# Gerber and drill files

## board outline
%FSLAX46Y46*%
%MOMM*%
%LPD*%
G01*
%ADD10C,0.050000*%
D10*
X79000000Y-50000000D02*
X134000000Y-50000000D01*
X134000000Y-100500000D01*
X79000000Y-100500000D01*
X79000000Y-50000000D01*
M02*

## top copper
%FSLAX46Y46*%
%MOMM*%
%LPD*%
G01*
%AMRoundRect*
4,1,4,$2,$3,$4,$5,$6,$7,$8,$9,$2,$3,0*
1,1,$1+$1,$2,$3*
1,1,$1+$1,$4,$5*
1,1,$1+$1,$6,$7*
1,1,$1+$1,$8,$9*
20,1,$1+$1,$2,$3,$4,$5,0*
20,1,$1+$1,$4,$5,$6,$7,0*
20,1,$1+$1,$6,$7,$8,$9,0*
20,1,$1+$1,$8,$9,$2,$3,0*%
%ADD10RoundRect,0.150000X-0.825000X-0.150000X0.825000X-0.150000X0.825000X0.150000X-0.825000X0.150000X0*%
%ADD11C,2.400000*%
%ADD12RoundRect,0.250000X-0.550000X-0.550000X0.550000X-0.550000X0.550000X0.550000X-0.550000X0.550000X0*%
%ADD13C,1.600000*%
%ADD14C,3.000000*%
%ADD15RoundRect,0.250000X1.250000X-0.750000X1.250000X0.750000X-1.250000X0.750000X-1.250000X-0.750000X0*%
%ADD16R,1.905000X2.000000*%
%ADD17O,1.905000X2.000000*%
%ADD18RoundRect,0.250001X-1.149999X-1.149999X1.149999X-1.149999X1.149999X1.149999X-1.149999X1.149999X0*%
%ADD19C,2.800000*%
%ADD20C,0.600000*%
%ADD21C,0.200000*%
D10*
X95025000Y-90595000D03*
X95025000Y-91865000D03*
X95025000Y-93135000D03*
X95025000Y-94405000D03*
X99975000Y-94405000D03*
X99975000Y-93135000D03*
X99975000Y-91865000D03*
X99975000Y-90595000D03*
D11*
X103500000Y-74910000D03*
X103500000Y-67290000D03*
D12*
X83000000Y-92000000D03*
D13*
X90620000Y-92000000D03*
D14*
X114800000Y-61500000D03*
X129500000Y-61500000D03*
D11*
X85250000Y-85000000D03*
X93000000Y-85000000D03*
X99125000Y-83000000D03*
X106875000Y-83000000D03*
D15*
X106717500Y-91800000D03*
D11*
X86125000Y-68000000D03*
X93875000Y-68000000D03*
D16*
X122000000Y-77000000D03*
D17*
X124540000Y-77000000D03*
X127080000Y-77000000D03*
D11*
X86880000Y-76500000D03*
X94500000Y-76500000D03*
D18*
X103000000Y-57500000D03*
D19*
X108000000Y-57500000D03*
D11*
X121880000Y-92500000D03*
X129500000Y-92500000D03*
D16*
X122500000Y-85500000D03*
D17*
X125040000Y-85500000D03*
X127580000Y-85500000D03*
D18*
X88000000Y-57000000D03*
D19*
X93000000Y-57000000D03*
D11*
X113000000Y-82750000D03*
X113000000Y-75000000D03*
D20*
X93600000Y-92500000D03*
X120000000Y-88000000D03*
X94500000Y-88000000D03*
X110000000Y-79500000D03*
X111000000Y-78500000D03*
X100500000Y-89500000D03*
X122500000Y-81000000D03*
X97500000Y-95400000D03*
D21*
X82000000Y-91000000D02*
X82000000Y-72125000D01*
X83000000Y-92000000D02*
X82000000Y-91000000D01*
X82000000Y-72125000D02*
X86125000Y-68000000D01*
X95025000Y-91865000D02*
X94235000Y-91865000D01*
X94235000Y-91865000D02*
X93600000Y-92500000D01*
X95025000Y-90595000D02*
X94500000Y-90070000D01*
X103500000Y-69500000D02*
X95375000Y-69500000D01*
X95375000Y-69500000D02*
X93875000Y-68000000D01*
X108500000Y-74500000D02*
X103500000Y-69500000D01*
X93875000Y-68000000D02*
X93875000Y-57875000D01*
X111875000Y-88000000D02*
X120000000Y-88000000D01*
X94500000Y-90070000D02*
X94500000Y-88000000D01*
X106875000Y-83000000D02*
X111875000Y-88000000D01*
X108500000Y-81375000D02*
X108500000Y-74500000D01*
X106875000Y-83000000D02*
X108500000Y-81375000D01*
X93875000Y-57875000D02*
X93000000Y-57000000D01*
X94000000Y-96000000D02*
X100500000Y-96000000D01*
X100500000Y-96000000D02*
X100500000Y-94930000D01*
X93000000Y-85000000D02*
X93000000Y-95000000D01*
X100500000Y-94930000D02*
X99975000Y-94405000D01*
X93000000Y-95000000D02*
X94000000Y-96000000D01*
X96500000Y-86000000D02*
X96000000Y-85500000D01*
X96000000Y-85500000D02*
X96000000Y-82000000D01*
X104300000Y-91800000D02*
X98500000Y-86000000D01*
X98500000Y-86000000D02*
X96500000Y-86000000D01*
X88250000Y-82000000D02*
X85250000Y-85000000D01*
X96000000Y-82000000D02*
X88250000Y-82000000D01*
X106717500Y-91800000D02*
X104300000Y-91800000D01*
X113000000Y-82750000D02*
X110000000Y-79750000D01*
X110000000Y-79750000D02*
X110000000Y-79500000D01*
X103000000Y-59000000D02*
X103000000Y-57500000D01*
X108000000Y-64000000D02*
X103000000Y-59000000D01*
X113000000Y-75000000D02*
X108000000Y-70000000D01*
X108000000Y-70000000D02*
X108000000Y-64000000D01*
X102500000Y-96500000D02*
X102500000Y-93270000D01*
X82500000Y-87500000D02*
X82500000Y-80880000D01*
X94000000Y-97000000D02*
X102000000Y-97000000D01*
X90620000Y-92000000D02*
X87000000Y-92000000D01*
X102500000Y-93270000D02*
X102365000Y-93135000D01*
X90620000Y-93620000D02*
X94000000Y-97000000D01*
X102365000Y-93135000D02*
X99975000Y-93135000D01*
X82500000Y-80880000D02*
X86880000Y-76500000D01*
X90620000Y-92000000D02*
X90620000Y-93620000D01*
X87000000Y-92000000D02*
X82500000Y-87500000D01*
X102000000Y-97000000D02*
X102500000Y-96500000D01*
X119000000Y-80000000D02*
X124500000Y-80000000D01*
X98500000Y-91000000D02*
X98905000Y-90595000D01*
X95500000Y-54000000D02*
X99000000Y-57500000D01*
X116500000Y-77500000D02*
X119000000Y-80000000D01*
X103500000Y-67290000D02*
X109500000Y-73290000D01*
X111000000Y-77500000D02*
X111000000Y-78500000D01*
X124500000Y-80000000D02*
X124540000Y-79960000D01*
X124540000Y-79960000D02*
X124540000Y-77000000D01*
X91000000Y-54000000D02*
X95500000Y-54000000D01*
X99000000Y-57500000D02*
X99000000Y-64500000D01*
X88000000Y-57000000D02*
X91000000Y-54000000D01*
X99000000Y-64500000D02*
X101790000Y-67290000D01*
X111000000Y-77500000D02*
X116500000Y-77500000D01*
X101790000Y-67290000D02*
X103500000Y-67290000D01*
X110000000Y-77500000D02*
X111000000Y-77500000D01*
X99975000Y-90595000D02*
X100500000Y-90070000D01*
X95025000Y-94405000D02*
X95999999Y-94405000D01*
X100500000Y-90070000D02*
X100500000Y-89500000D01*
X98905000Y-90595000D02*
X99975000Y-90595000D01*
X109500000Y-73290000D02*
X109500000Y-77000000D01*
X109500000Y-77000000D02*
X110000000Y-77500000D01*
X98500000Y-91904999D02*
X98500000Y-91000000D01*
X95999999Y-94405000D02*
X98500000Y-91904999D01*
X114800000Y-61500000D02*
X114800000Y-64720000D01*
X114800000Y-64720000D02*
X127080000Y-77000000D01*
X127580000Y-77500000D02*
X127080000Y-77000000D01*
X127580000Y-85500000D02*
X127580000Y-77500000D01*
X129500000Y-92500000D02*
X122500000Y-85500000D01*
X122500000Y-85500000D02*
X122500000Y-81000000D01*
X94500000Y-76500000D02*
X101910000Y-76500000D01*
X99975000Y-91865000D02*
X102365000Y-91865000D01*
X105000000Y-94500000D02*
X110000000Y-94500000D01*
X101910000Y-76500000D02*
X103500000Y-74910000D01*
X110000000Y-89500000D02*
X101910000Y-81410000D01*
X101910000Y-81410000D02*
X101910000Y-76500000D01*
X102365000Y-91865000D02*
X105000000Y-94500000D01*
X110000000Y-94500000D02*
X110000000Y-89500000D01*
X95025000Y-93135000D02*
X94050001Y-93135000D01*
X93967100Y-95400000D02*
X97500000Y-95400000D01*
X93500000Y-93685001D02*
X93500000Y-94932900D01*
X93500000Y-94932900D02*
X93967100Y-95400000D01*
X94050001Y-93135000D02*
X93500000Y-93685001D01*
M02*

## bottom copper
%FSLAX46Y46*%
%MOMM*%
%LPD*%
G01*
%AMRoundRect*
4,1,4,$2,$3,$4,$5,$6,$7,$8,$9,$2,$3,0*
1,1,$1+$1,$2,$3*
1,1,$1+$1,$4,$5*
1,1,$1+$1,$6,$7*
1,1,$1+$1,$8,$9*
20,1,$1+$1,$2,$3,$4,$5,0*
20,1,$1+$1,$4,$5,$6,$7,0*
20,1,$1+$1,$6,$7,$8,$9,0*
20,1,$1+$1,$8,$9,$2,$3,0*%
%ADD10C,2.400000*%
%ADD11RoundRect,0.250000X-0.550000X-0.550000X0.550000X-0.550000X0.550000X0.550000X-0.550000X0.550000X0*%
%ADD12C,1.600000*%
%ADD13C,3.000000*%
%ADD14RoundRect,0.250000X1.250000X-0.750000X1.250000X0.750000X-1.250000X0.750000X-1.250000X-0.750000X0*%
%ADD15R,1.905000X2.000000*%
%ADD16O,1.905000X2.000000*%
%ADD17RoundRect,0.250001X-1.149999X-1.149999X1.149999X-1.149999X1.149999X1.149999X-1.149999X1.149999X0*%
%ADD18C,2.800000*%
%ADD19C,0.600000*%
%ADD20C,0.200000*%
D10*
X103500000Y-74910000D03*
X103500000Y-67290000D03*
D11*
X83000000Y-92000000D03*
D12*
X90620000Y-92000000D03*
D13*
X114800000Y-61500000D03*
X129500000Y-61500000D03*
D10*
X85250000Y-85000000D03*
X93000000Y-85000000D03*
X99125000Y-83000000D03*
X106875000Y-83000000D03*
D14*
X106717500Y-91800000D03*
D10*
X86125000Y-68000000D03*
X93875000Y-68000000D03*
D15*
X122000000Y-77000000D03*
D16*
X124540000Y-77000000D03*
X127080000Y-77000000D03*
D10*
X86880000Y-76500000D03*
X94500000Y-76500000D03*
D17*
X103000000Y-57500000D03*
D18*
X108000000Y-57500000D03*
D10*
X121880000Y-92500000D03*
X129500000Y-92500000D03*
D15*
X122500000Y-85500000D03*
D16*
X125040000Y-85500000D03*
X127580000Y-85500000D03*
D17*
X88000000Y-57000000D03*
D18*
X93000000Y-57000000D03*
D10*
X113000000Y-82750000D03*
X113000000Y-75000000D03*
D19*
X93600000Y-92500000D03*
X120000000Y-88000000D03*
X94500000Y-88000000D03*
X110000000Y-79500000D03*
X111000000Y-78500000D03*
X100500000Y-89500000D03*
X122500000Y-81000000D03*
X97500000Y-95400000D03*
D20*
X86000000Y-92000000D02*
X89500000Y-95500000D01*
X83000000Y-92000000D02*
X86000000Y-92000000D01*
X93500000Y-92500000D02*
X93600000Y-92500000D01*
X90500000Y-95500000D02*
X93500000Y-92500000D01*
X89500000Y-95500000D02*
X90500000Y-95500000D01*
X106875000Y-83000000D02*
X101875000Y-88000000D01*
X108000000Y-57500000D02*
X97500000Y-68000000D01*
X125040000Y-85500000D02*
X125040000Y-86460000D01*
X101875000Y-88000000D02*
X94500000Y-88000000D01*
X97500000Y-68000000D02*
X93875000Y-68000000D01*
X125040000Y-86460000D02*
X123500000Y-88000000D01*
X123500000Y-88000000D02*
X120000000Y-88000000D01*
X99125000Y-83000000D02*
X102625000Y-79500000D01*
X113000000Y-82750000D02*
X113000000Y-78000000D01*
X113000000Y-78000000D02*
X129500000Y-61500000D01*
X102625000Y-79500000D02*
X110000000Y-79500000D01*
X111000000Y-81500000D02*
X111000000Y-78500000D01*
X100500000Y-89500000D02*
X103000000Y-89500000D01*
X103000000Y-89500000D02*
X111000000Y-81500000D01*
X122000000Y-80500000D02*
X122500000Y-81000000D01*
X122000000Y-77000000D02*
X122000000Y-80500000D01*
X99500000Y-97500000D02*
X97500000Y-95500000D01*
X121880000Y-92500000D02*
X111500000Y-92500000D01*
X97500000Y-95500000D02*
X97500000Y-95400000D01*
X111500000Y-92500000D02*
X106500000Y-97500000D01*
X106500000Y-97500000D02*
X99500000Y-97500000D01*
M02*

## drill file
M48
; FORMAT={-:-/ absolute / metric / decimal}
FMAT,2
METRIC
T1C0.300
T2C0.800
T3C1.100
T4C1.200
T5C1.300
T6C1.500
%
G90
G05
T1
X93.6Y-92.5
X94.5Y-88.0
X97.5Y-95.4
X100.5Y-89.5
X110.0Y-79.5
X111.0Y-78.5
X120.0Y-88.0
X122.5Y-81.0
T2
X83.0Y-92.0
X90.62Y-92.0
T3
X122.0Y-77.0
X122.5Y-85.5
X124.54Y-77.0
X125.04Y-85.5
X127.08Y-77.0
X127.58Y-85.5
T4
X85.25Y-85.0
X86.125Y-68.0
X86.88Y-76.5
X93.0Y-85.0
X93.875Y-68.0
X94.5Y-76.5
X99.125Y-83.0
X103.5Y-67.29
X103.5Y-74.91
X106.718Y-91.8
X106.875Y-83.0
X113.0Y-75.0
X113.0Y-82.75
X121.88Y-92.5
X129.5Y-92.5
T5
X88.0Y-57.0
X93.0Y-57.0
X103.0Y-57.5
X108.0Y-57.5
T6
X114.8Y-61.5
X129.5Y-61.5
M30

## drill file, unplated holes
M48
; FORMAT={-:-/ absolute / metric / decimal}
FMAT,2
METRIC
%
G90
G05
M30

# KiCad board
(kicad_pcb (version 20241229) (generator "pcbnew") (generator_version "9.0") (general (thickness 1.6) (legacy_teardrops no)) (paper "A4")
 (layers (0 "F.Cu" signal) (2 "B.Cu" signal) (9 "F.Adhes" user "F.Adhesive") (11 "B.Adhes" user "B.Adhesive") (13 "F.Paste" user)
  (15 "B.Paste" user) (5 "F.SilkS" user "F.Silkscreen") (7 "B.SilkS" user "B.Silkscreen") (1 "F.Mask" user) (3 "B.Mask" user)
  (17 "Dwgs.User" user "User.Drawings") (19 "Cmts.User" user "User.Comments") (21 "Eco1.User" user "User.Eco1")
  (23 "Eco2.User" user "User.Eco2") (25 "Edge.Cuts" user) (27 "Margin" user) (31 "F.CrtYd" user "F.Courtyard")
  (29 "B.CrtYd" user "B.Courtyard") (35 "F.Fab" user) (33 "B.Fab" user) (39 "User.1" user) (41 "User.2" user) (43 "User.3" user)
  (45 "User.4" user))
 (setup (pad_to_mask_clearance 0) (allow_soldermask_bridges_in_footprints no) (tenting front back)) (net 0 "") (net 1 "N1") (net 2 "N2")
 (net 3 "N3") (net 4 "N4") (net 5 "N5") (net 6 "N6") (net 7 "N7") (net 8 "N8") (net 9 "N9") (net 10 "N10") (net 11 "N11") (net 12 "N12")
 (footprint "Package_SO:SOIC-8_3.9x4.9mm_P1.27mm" (layer "F.Cu") (at 97.5 92.5)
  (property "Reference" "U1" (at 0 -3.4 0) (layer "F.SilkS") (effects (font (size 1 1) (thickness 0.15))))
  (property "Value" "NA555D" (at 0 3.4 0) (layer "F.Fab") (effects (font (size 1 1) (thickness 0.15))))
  (pad "1" smd roundrect (at -2.475 -1.905) (size 1.95 0.6) (layers "F.Cu" "F.Mask" "F.Paste") (roundrect_rratio 0.25) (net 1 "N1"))
  (pad "2" smd roundrect (at -2.475 -0.635) (size 1.95 0.6) (layers "F.Cu" "F.Mask" "F.Paste") (roundrect_rratio 0.25) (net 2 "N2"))
  (pad "3" smd roundrect (at -2.475 0.635) (size 1.95 0.6) (layers "F.Cu" "F.Mask" "F.Paste") (roundrect_rratio 0.25) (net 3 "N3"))
  (pad "4" smd roundrect (at -2.475 1.905) (size 1.95 0.6) (layers "F.Cu" "F.Mask" "F.Paste") (roundrect_rratio 0.25) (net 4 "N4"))
  (pad "5" smd roundrect (at 2.475 1.905) (size 1.95 0.6) (layers "F.Cu" "F.Mask" "F.Paste") (roundrect_rratio 0.25) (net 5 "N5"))
  (pad "6" smd roundrect (at 2.475 0.635) (size 1.95 0.6) (layers "F.Cu" "F.Mask" "F.Paste") (roundrect_rratio 0.25) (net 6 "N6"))
  (pad "7" smd roundrect (at 2.475 -0.635) (size 1.95 0.6) (layers "F.Cu" "F.Mask" "F.Paste") (roundrect_rratio 0.25) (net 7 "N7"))
  (pad "8" smd roundrect (at 2.475 -1.905) (size 1.95 0.6) (layers "F.Cu" "F.Mask" "F.Paste") (roundrect_rratio 0.25) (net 4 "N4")))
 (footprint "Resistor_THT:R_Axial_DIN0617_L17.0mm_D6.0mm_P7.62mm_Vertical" (layer "F.Cu") (at 103.5 74.91 90)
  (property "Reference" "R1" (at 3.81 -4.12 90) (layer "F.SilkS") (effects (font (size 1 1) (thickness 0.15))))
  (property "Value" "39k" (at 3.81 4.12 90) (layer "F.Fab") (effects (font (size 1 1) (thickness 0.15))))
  (pad "1" thru_hole circle (at 0 0 90) (size 2.4 2.4) (drill 1.2) (layers "*.Cu" "*.Mask") (remove_unused_layers no) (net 7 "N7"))
  (pad "2" thru_hole circle (at 7.62 0 90) (size 2.4 2.4) (drill 1.2) (layers "*.Cu" "*.Mask") (remove_unused_layers no) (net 4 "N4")))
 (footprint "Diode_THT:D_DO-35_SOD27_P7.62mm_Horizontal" (layer "F.Cu") (at 83 92)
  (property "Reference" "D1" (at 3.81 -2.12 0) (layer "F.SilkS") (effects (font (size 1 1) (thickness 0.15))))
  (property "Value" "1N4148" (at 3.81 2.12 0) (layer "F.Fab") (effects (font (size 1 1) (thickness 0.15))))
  (pad "1" thru_hole roundrect (at 0 0) (size 1.6 1.6) (drill 0.8) (layers "*.Cu" "*.Mask") (remove_unused_layers no)
   (roundrect_rratio 0.15625) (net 2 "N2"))
  (pad "2" thru_hole circle (at 7.62 0) (size 1.6 1.6) (drill 0.8) (layers "*.Cu" "*.Mask") (remove_unused_layers no) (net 6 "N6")))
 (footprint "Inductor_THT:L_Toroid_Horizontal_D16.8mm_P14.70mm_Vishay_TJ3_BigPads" (layer "F.Cu") (at 114.8 61.5)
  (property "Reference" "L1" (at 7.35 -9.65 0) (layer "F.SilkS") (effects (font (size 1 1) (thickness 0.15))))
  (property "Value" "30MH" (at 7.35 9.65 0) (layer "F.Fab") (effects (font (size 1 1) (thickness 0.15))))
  (pad "1" thru_hole circle (at 0 0) (size 3 3) (drill 1.5) (layers "*.Cu" "*.Mask") (remove_unused_layers no) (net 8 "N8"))
  (pad "2" thru_hole circle (at 14.7 0) (size 3 3) (drill 1.5) (layers "*.Cu" "*.Mask") (remove_unused_layers no) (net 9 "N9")))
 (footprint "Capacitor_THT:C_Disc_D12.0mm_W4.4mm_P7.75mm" (layer "F.Cu") (at 85.25 85)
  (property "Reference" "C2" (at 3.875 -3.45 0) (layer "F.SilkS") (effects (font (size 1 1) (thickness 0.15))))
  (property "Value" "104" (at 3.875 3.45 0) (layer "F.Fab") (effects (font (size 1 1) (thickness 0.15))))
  (pad "1" thru_hole circle (at 0 0) (size 2.4 2.4) (drill 1.2) (layers "*.Cu" "*.Mask") (remove_unused_layers no) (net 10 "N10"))
  (pad "2" thru_hole circle (at 7.75 0) (size 2.4 2.4) (drill 1.2) (layers "*.Cu" "*.Mask") (remove_unused_layers no) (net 5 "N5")))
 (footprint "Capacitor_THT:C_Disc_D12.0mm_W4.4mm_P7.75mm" (layer "F.Cu") (at 99.125 83)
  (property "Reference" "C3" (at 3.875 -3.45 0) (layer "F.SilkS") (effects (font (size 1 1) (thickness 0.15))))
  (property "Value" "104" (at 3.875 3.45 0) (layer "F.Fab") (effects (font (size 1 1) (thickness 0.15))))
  (pad "1" thru_hole circle (at 0 0) (size 2.4 2.4) (drill 1.2) (layers "*.Cu" "*.Mask") (remove_unused_layers no) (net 9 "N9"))
  (pad "2" thru_hole circle (at 7.75 0) (size 2.4 2.4) (drill 1.2) (layers "*.Cu" "*.Mask") (remove_unused_layers no) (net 1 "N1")))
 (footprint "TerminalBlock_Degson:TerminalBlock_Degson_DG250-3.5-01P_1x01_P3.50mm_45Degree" (layer "F.Cu") (at 106.7175 91.8 90)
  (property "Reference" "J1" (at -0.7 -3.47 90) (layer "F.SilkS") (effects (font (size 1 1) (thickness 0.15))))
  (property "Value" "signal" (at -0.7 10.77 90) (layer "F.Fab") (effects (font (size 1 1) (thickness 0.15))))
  (pad "1" thru_hole roundrect (at 0 0 90) (size 2 3) (drill 1.2) (layers "*.Cu" "*.Mask") (remove_unused_layers no)
   (roundrect_rratio 0.125) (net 10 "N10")))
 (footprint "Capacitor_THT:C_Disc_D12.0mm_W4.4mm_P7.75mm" (layer "F.Cu") (at 86.125 68)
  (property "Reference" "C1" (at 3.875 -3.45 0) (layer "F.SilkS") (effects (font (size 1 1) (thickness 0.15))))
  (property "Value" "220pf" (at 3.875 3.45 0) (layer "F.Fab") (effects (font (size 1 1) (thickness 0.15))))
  (pad "1" thru_hole circle (at 0 0) (size 2.4 2.4) (drill 1.2) (layers "*.Cu" "*.Mask") (remove_unused_layers no) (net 2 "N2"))
  (pad "2" thru_hole circle (at 7.75 0) (size 2.4 2.4) (drill 1.2) (layers "*.Cu" "*.Mask") (remove_unused_layers no) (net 1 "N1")))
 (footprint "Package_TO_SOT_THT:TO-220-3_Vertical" (layer "F.Cu") (at 122 77)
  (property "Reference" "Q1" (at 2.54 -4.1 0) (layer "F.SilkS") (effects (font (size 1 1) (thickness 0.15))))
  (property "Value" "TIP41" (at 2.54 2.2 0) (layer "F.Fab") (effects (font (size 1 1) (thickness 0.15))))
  (pad "1" thru_hole rect (at 0 0) (size 1.905 2) (drill 1.1) (layers "*.Cu" "*.Mask") (remove_unused_layers no) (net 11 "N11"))
  (pad "2" thru_hole oval (at 2.54 0) (size 1.905 2) (drill 1.1) (layers "*.Cu" "*.Mask") (remove_unused_layers no) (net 4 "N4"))
  (pad "3" thru_hole oval (at 5.08 0) (size 1.905 2) (drill 1.1) (layers "*.Cu" "*.Mask") (remove_unused_layers no) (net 8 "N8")))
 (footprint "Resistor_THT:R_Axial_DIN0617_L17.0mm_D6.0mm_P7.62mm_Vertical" (layer "F.Cu") (at 86.88 76.5)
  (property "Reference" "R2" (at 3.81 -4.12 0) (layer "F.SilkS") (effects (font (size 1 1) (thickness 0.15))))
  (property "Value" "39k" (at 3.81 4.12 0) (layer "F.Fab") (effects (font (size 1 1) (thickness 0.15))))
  (pad "1" thru_hole circle (at 0 0) (size 2.4 2.4) (drill 1.2) (layers "*.Cu" "*.Mask") (remove_unused_layers no) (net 6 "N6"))
  (pad "2" thru_hole circle (at 7.62 0) (size 2.4 2.4) (drill 1.2) (layers "*.Cu" "*.Mask") (remove_unused_layers no) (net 7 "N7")))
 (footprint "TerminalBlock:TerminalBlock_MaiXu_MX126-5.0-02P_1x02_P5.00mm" (layer "F.Cu") (at 103 57.5)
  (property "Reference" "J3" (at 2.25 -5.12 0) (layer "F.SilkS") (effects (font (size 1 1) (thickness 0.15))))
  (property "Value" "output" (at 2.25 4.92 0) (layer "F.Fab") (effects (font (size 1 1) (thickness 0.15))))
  (pad "1" thru_hole roundrect (at 0 0) (size 2.8 2.8) (drill 1.3) (layers "*.Cu" "*.Mask") (remove_unused_layers no)
   (roundrect_rratio 0.089286) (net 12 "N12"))
  (pad "2" thru_hole circle (at 5 0) (size 2.8 2.8) (drill 1.3) (layers "*.Cu" "*.Mask") (remove_unused_layers no) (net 1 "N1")))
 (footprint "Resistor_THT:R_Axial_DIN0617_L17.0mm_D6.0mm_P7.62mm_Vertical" (layer "F.Cu") (at 121.88 92.5)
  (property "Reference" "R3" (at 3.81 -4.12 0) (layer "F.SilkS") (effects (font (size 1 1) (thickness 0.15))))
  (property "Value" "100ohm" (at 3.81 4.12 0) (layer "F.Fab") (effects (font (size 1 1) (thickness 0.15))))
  (pad "1" thru_hole circle (at 0 0) (size 2.4 2.4) (drill 1.2) (layers "*.Cu" "*.Mask") (remove_unused_layers no) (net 3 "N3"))
  (pad "2" thru_hole circle (at 7.62 0) (size 2.4 2.4) (drill 1.2) (layers "*.Cu" "*.Mask") (remove_unused_layers no) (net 11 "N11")))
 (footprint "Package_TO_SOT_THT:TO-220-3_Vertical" (layer "F.Cu") (at 122.5 85.5)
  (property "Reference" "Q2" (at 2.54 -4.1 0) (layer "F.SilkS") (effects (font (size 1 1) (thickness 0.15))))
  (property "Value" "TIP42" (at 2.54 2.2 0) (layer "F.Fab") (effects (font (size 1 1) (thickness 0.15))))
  (pad "1" thru_hole rect (at 0 0) (size 1.905 2) (drill 1.1) (layers "*.Cu" "*.Mask") (remove_unused_layers no) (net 11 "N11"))
  (pad "2" thru_hole oval (at 2.54 0) (size 1.905 2) (drill 1.1) (layers "*.Cu" "*.Mask") (remove_unused_layers no) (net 1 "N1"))
  (pad "3" thru_hole oval (at 5.08 0) (size 1.905 2) (drill 1.1) (layers "*.Cu" "*.Mask") (remove_unused_layers no) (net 8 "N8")))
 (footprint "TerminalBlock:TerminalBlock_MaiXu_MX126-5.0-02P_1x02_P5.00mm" (layer "F.Cu") (at 88 57)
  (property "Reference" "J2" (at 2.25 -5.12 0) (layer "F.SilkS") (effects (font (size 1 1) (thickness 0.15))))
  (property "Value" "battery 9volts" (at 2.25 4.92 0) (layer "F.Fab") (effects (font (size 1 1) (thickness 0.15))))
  (pad "1" thru_hole roundrect (at 0 0) (size 2.8 2.8) (drill 1.3) (layers "*.Cu" "*.Mask") (remove_unused_layers no)
   (roundrect_rratio 0.089286) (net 4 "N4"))
  (pad "2" thru_hole circle (at 5 0) (size 2.8 2.8) (drill 1.3) (layers "*.Cu" "*.Mask") (remove_unused_layers no) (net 1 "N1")))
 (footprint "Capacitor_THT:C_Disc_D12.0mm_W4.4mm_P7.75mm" (layer "F.Cu") (at 113 82.75 90)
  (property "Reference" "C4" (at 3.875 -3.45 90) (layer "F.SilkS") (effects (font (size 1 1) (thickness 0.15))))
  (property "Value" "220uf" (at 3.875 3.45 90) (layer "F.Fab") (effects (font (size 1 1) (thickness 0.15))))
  (pad "1" thru_hole circle (at 0 0 90) (size 2.4 2.4) (drill 1.2) (layers "*.Cu" "*.Mask") (remove_unused_layers no) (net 9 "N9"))
  (pad "2" thru_hole circle (at 7.75 0 90) (size 2.4 2.4) (drill 1.2) (layers "*.Cu" "*.Mask") (remove_unused_layers no) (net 12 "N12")))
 (gr_rect (start 79 50) (end 134 100.5) (stroke (width 0.05) (type default)) (fill no) (layer "Edge.Cuts"))
 (segment (start 82 91) (end 82 72.125) (width 0.2) (layer "F.Cu") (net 2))
 (segment (start 83 92) (end 82 91) (width 0.2) (layer "F.Cu") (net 2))
 (segment (start 82 72.125) (end 86.125 68) (width 0.2) (layer "F.Cu") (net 2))
 (segment (start 95.025 91.865) (end 94.235 91.865) (width 0.2) (layer "F.Cu") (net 2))
 (segment (start 94.235 91.865) (end 93.6 92.5) (width 0.2) (layer "F.Cu") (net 2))
 (via (at 93.6 92.5) (size 0.6) (drill 0.3) (layers "F.Cu" "B.Cu") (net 2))
 (segment (start 86 92) (end 89.5 95.5) (width 0.2) (layer "B.Cu") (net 2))
 (segment (start 83 92) (end 86 92) (width 0.2) (layer "B.Cu") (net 2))
 (segment (start 93.5 92.5) (end 93.6 92.5) (width 0.2) (layer "B.Cu") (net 2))
 (segment (start 90.5 95.5) (end 93.5 92.5) (width 0.2) (layer "B.Cu") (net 2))
 (segment (start 89.5 95.5) (end 90.5 95.5) (width 0.2) (layer "B.Cu") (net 2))
 (segment (start 95.025 90.595) (end 94.5 90.07) (width 0.2) (layer "F.Cu") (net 1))
 (segment (start 103.5 69.5) (end 95.375 69.5) (width 0.2) (layer "F.Cu") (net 1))
 (segment (start 95.375 69.5) (end 93.875 68) (width 0.2) (layer "F.Cu") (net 1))
 (segment (start 108.5 74.5) (end 103.5 69.5) (width 0.2) (layer "F.Cu") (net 1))
 (segment (start 93.875 68) (end 93.875 57.875) (width 0.2) (layer "F.Cu") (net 1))
 (segment (start 111.875 88) (end 120 88) (width 0.2) (layer "F.Cu") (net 1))
 (segment (start 94.5 90.07) (end 94.5 88) (width 0.2) (layer "F.Cu") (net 1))
 (segment (start 106.875 83) (end 111.875 88) (width 0.2) (layer "F.Cu") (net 1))
 (segment (start 108.5 81.375) (end 108.5 74.5) (width 0.2) (layer "F.Cu") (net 1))
 (segment (start 106.875 83) (end 108.5 81.375) (width 0.2) (layer "F.Cu") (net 1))
 (segment (start 93.875 57.875) (end 93 57) (width 0.2) (layer "F.Cu") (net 1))
 (via (at 120 88) (size 0.6) (drill 0.3) (layers "F.Cu" "B.Cu") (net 1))
 (via (at 94.5 88) (size 0.6) (drill 0.3) (layers "F.Cu" "B.Cu") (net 1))
 (segment (start 106.875 83) (end 101.875 88) (width 0.2) (layer "B.Cu") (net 1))
 (segment (start 108 57.5) (end 97.5 68) (width 0.2) (layer "B.Cu") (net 1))
 (segment (start 125.04 85.5) (end 125.04 86.46) (width 0.2) (layer "B.Cu") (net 1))
 (segment (start 101.875 88) (end 94.5 88) (width 0.2) (layer "B.Cu") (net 1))
 (segment (start 97.5 68) (end 93.875 68) (width 0.2) (layer "B.Cu") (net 1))
 (segment (start 125.04 86.46) (end 123.5 88) (width 0.2) (layer "B.Cu") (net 1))
 (segment (start 123.5 88) (end 120 88) (width 0.2) (layer "B.Cu") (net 1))
 (segment (start 94 96) (end 100.5 96) (width 0.2) (layer "F.Cu") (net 5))
 (segment (start 100.5 96) (end 100.5 94.93) (width 0.2) (layer "F.Cu") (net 5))
 (segment (start 93 85) (end 93 95) (width 0.2) (layer "F.Cu") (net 5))
 (segment (start 100.5 94.93) (end 99.975 94.405) (width 0.2) (layer "F.Cu") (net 5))
 (segment (start 93 95) (end 94 96) (width 0.2) (layer "F.Cu") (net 5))
 (segment (start 96.5 86) (end 96 85.5) (width 0.2) (layer "F.Cu") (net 10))
 (segment (start 96 85.5) (end 96 82) (width 0.2) (layer "F.Cu") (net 10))
 (segment (start 104.3 91.8) (end 98.5 86) (width 0.2) (layer "F.Cu") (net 10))
 (segment (start 98.5 86) (end 96.5 86) (width 0.2) (layer "F.Cu") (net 10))
 (segment (start 88.25 82) (end 85.25 85) (width 0.2) (layer "F.Cu") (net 10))
 (segment (start 96 82) (end 88.25 82) (width 0.2) (layer "F.Cu") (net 10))
 (segment (start 106.7175 91.8) (end 104.3 91.8) (width 0.2) (layer "F.Cu") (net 10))
 (segment (start 113 82.75) (end 110 79.75) (width 0.2) (layer "F.Cu") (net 9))
 (segment (start 110 79.75) (end 110 79.5) (width 0.2) (layer "F.Cu") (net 9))
 (via (at 110 79.5) (size 0.6) (drill 0.3) (layers "F.Cu" "B.Cu") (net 9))
 (segment (start 99.125 83) (end 102.625 79.5) (width 0.2) (layer "B.Cu") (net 9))
 (segment (start 113 82.75) (end 113 78) (width 0.2) (layer "B.Cu") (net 9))
 (segment (start 113 78) (end 129.5 61.5) (width 0.2) (layer "B.Cu") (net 9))
 (segment (start 102.625 79.5) (end 110 79.5) (width 0.2) (layer "B.Cu") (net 9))
 (segment (start 103 59) (end 103 57.5) (width 0.2) (layer "F.Cu") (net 12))
 (segment (start 108 64) (end 103 59) (width 0.2) (layer "F.Cu") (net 12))
 (segment (start 113 75) (end 108 70) (width 0.2) (layer "F.Cu") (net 12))
 (segment (start 108 70) (end 108 64) (width 0.2) (layer "F.Cu") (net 12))
 (segment (start 102.5 96.5) (end 102.5 93.27) (width 0.2) (layer "F.Cu") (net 6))
 (segment (start 82.5 87.5) (end 82.5 80.88) (width 0.2) (layer "F.Cu") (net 6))
 (segment (start 94 97) (end 102 97) (width 0.2) (layer "F.Cu") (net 6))
 (segment (start 90.62 92) (end 87 92) (width 0.2) (layer "F.Cu") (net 6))
 (segment (start 102.5 93.27) (end 102.365 93.135) (width 0.2) (layer "F.Cu") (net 6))
 (segment (start 90.62 93.62) (end 94 97) (width 0.2) (layer "F.Cu") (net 6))
 (segment (start 102.365 93.135) (end 99.975 93.135) (width 0.2) (layer "F.Cu") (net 6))
 (segment (start 82.5 80.88) (end 86.88 76.5) (width 0.2) (layer "F.Cu") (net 6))
 (segment (start 90.62 92) (end 90.62 93.62) (width 0.2) (layer "F.Cu") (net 6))
 (segment (start 87 92) (end 82.5 87.5) (width 0.2) (layer "F.Cu") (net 6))
 (segment (start 102 97) (end 102.5 96.5) (width 0.2) (layer "F.Cu") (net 6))
 (segment (start 119 80) (end 124.5 80) (width 0.2) (layer "F.Cu") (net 4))
 (segment (start 98.5 91) (end 98.905 90.595) (width 0.2) (layer "F.Cu") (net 4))
 (segment (start 95.5 54) (end 99 57.5) (width 0.2) (layer "F.Cu") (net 4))
 (segment (start 116.5 77.5) (end 119 80) (width 0.2) (layer "F.Cu") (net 4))
 (segment (start 103.5 67.29) (end 109.5 73.29) (width 0.2) (layer "F.Cu") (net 4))
 (segment (start 111 77.5) (end 111 78.5) (width 0.2) (layer "F.Cu") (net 4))
 (segment (start 124.5 80) (end 124.54 79.96) (width 0.2) (layer "F.Cu") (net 4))
 (segment (start 124.54 79.96) (end 124.54 77) (width 0.2) (layer "F.Cu") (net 4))
 (segment (start 91 54) (end 95.5 54) (width 0.2) (layer "F.Cu") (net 4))
 (segment (start 99 57.5) (end 99 64.5) (width 0.2) (layer "F.Cu") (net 4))
 (segment (start 88 57) (end 91 54) (width 0.2) (layer "F.Cu") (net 4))
 (segment (start 99 64.5) (end 101.79 67.29) (width 0.2) (layer "F.Cu") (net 4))
 (segment (start 111 77.5) (end 116.5 77.5) (width 0.2) (layer "F.Cu") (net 4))
 (segment (start 101.79 67.29) (end 103.5 67.29) (width 0.2) (layer "F.Cu") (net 4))
 (segment (start 110 77.5) (end 111 77.5) (width 0.2) (layer "F.Cu") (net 4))
 (segment (start 99.975 90.595) (end 100.5 90.07) (width 0.2) (layer "F.Cu") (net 4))
 (segment (start 95.025 94.405) (end 95.999999 94.405) (width 0.2) (layer "F.Cu") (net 4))
 (segment (start 100.5 90.07) (end 100.5 89.5) (width 0.2) (layer "F.Cu") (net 4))
 (segment (start 98.905 90.595) (end 99.975 90.595) (width 0.2) (layer "F.Cu") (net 4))
 (segment (start 109.5 73.29) (end 109.5 77) (width 0.2) (layer "F.Cu") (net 4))
 (segment (start 109.5 77) (end 110 77.5) (width 0.2) (layer "F.Cu") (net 4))
 (segment (start 98.5 91.904999) (end 98.5 91) (width 0.2) (layer "F.Cu") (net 4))
 (segment (start 95.999999 94.405) (end 98.5 91.904999) (width 0.2) (layer "F.Cu") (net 4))
 (via (at 111 78.5) (size 0.6) (drill 0.3) (layers "F.Cu" "B.Cu") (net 4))
 (via (at 100.5 89.5) (size 0.6) (drill 0.3) (layers "F.Cu" "B.Cu") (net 4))
 (segment (start 111 81.5) (end 111 78.5) (width 0.2) (layer "B.Cu") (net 4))
 (segment (start 100.5 89.5) (end 103 89.5) (width 0.2) (layer "B.Cu") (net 4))
 (segment (start 103 89.5) (end 111 81.5) (width 0.2) (layer "B.Cu") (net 4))
 (segment (start 114.8 61.5) (end 114.8 64.72) (width 0.2) (layer "F.Cu") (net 8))
 (segment (start 114.8 64.72) (end 127.08 77) (width 0.2) (layer "F.Cu") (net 8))
 (segment (start 127.58 77.5) (end 127.08 77) (width 0.2) (layer "F.Cu") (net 8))
 (segment (start 127.58 85.5) (end 127.58 77.5) (width 0.2) (layer "F.Cu") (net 8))
 (segment (start 129.5 92.5) (end 122.5 85.5) (width 0.2) (layer "F.Cu") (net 11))
 (segment (start 122.5 85.5) (end 122.5 81) (width 0.2) (layer "F.Cu") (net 11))
 (via (at 122.5 81) (size 0.6) (drill 0.3) (layers "F.Cu" "B.Cu") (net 11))
 (segment (start 122 80.5) (end 122.5 81) (width 0.2) (layer "B.Cu") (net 11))
 (segment (start 122 77) (end 122 80.5) (width 0.2) (layer "B.Cu") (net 11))
 (segment (start 94.5 76.5) (end 101.91 76.5) (width 0.2) (layer "F.Cu") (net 7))
 (segment (start 99.975 91.865) (end 102.365 91.865) (width 0.2) (layer "F.Cu") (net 7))
 (segment (start 105 94.5) (end 110 94.5) (width 0.2) (layer "F.Cu") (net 7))
 (segment (start 101.91 76.5) (end 103.5 74.91) (width 0.2) (layer "F.Cu") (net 7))
 (segment (start 110 89.5) (end 101.91 81.41) (width 0.2) (layer "F.Cu") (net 7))
 (segment (start 101.91 81.41) (end 101.91 76.5) (width 0.2) (layer "F.Cu") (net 7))
 (segment (start 102.365 91.865) (end 105 94.5) (width 0.2) (layer "F.Cu") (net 7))
 (segment (start 110 94.5) (end 110 89.5) (width 0.2) (layer "F.Cu") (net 7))
 (segment (start 95.025 93.135) (end 94.050001 93.135) (width 0.2) (layer "F.Cu") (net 3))
 (segment (start 93.9671 95.4) (end 97.5 95.4) (width 0.2) (layer "F.Cu") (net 3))
 (segment (start 93.5 93.685001) (end 93.5 94.9329) (width 0.2) (layer "F.Cu") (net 3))
 (segment (start 93.5 94.9329) (end 93.9671 95.4) (width 0.2) (layer "F.Cu") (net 3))
 (segment (start 94.050001 93.135) (end 93.5 93.685001) (width 0.2) (layer "F.Cu") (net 3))
 (via (at 97.5 95.4) (size 0.6) (drill 0.3) (layers "F.Cu" "B.Cu") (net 3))
 (segment (start 99.5 97.5) (end 97.5 95.5) (width 0.2) (layer "B.Cu") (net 3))
 (segment (start 121.88 92.5) (end 111.5 92.5) (width 0.2) (layer "B.Cu") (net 3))
 (segment (start 97.5 95.5) (end 97.5 95.4) (width 0.2) (layer "B.Cu") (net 3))
 (segment (start 111.5 92.5) (end 106.5 97.5) (width 0.2) (layer "B.Cu") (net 3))
 (segment (start 106.5 97.5) (end 99.5 97.5) (width 0.2) (layer "B.Cu") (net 3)))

